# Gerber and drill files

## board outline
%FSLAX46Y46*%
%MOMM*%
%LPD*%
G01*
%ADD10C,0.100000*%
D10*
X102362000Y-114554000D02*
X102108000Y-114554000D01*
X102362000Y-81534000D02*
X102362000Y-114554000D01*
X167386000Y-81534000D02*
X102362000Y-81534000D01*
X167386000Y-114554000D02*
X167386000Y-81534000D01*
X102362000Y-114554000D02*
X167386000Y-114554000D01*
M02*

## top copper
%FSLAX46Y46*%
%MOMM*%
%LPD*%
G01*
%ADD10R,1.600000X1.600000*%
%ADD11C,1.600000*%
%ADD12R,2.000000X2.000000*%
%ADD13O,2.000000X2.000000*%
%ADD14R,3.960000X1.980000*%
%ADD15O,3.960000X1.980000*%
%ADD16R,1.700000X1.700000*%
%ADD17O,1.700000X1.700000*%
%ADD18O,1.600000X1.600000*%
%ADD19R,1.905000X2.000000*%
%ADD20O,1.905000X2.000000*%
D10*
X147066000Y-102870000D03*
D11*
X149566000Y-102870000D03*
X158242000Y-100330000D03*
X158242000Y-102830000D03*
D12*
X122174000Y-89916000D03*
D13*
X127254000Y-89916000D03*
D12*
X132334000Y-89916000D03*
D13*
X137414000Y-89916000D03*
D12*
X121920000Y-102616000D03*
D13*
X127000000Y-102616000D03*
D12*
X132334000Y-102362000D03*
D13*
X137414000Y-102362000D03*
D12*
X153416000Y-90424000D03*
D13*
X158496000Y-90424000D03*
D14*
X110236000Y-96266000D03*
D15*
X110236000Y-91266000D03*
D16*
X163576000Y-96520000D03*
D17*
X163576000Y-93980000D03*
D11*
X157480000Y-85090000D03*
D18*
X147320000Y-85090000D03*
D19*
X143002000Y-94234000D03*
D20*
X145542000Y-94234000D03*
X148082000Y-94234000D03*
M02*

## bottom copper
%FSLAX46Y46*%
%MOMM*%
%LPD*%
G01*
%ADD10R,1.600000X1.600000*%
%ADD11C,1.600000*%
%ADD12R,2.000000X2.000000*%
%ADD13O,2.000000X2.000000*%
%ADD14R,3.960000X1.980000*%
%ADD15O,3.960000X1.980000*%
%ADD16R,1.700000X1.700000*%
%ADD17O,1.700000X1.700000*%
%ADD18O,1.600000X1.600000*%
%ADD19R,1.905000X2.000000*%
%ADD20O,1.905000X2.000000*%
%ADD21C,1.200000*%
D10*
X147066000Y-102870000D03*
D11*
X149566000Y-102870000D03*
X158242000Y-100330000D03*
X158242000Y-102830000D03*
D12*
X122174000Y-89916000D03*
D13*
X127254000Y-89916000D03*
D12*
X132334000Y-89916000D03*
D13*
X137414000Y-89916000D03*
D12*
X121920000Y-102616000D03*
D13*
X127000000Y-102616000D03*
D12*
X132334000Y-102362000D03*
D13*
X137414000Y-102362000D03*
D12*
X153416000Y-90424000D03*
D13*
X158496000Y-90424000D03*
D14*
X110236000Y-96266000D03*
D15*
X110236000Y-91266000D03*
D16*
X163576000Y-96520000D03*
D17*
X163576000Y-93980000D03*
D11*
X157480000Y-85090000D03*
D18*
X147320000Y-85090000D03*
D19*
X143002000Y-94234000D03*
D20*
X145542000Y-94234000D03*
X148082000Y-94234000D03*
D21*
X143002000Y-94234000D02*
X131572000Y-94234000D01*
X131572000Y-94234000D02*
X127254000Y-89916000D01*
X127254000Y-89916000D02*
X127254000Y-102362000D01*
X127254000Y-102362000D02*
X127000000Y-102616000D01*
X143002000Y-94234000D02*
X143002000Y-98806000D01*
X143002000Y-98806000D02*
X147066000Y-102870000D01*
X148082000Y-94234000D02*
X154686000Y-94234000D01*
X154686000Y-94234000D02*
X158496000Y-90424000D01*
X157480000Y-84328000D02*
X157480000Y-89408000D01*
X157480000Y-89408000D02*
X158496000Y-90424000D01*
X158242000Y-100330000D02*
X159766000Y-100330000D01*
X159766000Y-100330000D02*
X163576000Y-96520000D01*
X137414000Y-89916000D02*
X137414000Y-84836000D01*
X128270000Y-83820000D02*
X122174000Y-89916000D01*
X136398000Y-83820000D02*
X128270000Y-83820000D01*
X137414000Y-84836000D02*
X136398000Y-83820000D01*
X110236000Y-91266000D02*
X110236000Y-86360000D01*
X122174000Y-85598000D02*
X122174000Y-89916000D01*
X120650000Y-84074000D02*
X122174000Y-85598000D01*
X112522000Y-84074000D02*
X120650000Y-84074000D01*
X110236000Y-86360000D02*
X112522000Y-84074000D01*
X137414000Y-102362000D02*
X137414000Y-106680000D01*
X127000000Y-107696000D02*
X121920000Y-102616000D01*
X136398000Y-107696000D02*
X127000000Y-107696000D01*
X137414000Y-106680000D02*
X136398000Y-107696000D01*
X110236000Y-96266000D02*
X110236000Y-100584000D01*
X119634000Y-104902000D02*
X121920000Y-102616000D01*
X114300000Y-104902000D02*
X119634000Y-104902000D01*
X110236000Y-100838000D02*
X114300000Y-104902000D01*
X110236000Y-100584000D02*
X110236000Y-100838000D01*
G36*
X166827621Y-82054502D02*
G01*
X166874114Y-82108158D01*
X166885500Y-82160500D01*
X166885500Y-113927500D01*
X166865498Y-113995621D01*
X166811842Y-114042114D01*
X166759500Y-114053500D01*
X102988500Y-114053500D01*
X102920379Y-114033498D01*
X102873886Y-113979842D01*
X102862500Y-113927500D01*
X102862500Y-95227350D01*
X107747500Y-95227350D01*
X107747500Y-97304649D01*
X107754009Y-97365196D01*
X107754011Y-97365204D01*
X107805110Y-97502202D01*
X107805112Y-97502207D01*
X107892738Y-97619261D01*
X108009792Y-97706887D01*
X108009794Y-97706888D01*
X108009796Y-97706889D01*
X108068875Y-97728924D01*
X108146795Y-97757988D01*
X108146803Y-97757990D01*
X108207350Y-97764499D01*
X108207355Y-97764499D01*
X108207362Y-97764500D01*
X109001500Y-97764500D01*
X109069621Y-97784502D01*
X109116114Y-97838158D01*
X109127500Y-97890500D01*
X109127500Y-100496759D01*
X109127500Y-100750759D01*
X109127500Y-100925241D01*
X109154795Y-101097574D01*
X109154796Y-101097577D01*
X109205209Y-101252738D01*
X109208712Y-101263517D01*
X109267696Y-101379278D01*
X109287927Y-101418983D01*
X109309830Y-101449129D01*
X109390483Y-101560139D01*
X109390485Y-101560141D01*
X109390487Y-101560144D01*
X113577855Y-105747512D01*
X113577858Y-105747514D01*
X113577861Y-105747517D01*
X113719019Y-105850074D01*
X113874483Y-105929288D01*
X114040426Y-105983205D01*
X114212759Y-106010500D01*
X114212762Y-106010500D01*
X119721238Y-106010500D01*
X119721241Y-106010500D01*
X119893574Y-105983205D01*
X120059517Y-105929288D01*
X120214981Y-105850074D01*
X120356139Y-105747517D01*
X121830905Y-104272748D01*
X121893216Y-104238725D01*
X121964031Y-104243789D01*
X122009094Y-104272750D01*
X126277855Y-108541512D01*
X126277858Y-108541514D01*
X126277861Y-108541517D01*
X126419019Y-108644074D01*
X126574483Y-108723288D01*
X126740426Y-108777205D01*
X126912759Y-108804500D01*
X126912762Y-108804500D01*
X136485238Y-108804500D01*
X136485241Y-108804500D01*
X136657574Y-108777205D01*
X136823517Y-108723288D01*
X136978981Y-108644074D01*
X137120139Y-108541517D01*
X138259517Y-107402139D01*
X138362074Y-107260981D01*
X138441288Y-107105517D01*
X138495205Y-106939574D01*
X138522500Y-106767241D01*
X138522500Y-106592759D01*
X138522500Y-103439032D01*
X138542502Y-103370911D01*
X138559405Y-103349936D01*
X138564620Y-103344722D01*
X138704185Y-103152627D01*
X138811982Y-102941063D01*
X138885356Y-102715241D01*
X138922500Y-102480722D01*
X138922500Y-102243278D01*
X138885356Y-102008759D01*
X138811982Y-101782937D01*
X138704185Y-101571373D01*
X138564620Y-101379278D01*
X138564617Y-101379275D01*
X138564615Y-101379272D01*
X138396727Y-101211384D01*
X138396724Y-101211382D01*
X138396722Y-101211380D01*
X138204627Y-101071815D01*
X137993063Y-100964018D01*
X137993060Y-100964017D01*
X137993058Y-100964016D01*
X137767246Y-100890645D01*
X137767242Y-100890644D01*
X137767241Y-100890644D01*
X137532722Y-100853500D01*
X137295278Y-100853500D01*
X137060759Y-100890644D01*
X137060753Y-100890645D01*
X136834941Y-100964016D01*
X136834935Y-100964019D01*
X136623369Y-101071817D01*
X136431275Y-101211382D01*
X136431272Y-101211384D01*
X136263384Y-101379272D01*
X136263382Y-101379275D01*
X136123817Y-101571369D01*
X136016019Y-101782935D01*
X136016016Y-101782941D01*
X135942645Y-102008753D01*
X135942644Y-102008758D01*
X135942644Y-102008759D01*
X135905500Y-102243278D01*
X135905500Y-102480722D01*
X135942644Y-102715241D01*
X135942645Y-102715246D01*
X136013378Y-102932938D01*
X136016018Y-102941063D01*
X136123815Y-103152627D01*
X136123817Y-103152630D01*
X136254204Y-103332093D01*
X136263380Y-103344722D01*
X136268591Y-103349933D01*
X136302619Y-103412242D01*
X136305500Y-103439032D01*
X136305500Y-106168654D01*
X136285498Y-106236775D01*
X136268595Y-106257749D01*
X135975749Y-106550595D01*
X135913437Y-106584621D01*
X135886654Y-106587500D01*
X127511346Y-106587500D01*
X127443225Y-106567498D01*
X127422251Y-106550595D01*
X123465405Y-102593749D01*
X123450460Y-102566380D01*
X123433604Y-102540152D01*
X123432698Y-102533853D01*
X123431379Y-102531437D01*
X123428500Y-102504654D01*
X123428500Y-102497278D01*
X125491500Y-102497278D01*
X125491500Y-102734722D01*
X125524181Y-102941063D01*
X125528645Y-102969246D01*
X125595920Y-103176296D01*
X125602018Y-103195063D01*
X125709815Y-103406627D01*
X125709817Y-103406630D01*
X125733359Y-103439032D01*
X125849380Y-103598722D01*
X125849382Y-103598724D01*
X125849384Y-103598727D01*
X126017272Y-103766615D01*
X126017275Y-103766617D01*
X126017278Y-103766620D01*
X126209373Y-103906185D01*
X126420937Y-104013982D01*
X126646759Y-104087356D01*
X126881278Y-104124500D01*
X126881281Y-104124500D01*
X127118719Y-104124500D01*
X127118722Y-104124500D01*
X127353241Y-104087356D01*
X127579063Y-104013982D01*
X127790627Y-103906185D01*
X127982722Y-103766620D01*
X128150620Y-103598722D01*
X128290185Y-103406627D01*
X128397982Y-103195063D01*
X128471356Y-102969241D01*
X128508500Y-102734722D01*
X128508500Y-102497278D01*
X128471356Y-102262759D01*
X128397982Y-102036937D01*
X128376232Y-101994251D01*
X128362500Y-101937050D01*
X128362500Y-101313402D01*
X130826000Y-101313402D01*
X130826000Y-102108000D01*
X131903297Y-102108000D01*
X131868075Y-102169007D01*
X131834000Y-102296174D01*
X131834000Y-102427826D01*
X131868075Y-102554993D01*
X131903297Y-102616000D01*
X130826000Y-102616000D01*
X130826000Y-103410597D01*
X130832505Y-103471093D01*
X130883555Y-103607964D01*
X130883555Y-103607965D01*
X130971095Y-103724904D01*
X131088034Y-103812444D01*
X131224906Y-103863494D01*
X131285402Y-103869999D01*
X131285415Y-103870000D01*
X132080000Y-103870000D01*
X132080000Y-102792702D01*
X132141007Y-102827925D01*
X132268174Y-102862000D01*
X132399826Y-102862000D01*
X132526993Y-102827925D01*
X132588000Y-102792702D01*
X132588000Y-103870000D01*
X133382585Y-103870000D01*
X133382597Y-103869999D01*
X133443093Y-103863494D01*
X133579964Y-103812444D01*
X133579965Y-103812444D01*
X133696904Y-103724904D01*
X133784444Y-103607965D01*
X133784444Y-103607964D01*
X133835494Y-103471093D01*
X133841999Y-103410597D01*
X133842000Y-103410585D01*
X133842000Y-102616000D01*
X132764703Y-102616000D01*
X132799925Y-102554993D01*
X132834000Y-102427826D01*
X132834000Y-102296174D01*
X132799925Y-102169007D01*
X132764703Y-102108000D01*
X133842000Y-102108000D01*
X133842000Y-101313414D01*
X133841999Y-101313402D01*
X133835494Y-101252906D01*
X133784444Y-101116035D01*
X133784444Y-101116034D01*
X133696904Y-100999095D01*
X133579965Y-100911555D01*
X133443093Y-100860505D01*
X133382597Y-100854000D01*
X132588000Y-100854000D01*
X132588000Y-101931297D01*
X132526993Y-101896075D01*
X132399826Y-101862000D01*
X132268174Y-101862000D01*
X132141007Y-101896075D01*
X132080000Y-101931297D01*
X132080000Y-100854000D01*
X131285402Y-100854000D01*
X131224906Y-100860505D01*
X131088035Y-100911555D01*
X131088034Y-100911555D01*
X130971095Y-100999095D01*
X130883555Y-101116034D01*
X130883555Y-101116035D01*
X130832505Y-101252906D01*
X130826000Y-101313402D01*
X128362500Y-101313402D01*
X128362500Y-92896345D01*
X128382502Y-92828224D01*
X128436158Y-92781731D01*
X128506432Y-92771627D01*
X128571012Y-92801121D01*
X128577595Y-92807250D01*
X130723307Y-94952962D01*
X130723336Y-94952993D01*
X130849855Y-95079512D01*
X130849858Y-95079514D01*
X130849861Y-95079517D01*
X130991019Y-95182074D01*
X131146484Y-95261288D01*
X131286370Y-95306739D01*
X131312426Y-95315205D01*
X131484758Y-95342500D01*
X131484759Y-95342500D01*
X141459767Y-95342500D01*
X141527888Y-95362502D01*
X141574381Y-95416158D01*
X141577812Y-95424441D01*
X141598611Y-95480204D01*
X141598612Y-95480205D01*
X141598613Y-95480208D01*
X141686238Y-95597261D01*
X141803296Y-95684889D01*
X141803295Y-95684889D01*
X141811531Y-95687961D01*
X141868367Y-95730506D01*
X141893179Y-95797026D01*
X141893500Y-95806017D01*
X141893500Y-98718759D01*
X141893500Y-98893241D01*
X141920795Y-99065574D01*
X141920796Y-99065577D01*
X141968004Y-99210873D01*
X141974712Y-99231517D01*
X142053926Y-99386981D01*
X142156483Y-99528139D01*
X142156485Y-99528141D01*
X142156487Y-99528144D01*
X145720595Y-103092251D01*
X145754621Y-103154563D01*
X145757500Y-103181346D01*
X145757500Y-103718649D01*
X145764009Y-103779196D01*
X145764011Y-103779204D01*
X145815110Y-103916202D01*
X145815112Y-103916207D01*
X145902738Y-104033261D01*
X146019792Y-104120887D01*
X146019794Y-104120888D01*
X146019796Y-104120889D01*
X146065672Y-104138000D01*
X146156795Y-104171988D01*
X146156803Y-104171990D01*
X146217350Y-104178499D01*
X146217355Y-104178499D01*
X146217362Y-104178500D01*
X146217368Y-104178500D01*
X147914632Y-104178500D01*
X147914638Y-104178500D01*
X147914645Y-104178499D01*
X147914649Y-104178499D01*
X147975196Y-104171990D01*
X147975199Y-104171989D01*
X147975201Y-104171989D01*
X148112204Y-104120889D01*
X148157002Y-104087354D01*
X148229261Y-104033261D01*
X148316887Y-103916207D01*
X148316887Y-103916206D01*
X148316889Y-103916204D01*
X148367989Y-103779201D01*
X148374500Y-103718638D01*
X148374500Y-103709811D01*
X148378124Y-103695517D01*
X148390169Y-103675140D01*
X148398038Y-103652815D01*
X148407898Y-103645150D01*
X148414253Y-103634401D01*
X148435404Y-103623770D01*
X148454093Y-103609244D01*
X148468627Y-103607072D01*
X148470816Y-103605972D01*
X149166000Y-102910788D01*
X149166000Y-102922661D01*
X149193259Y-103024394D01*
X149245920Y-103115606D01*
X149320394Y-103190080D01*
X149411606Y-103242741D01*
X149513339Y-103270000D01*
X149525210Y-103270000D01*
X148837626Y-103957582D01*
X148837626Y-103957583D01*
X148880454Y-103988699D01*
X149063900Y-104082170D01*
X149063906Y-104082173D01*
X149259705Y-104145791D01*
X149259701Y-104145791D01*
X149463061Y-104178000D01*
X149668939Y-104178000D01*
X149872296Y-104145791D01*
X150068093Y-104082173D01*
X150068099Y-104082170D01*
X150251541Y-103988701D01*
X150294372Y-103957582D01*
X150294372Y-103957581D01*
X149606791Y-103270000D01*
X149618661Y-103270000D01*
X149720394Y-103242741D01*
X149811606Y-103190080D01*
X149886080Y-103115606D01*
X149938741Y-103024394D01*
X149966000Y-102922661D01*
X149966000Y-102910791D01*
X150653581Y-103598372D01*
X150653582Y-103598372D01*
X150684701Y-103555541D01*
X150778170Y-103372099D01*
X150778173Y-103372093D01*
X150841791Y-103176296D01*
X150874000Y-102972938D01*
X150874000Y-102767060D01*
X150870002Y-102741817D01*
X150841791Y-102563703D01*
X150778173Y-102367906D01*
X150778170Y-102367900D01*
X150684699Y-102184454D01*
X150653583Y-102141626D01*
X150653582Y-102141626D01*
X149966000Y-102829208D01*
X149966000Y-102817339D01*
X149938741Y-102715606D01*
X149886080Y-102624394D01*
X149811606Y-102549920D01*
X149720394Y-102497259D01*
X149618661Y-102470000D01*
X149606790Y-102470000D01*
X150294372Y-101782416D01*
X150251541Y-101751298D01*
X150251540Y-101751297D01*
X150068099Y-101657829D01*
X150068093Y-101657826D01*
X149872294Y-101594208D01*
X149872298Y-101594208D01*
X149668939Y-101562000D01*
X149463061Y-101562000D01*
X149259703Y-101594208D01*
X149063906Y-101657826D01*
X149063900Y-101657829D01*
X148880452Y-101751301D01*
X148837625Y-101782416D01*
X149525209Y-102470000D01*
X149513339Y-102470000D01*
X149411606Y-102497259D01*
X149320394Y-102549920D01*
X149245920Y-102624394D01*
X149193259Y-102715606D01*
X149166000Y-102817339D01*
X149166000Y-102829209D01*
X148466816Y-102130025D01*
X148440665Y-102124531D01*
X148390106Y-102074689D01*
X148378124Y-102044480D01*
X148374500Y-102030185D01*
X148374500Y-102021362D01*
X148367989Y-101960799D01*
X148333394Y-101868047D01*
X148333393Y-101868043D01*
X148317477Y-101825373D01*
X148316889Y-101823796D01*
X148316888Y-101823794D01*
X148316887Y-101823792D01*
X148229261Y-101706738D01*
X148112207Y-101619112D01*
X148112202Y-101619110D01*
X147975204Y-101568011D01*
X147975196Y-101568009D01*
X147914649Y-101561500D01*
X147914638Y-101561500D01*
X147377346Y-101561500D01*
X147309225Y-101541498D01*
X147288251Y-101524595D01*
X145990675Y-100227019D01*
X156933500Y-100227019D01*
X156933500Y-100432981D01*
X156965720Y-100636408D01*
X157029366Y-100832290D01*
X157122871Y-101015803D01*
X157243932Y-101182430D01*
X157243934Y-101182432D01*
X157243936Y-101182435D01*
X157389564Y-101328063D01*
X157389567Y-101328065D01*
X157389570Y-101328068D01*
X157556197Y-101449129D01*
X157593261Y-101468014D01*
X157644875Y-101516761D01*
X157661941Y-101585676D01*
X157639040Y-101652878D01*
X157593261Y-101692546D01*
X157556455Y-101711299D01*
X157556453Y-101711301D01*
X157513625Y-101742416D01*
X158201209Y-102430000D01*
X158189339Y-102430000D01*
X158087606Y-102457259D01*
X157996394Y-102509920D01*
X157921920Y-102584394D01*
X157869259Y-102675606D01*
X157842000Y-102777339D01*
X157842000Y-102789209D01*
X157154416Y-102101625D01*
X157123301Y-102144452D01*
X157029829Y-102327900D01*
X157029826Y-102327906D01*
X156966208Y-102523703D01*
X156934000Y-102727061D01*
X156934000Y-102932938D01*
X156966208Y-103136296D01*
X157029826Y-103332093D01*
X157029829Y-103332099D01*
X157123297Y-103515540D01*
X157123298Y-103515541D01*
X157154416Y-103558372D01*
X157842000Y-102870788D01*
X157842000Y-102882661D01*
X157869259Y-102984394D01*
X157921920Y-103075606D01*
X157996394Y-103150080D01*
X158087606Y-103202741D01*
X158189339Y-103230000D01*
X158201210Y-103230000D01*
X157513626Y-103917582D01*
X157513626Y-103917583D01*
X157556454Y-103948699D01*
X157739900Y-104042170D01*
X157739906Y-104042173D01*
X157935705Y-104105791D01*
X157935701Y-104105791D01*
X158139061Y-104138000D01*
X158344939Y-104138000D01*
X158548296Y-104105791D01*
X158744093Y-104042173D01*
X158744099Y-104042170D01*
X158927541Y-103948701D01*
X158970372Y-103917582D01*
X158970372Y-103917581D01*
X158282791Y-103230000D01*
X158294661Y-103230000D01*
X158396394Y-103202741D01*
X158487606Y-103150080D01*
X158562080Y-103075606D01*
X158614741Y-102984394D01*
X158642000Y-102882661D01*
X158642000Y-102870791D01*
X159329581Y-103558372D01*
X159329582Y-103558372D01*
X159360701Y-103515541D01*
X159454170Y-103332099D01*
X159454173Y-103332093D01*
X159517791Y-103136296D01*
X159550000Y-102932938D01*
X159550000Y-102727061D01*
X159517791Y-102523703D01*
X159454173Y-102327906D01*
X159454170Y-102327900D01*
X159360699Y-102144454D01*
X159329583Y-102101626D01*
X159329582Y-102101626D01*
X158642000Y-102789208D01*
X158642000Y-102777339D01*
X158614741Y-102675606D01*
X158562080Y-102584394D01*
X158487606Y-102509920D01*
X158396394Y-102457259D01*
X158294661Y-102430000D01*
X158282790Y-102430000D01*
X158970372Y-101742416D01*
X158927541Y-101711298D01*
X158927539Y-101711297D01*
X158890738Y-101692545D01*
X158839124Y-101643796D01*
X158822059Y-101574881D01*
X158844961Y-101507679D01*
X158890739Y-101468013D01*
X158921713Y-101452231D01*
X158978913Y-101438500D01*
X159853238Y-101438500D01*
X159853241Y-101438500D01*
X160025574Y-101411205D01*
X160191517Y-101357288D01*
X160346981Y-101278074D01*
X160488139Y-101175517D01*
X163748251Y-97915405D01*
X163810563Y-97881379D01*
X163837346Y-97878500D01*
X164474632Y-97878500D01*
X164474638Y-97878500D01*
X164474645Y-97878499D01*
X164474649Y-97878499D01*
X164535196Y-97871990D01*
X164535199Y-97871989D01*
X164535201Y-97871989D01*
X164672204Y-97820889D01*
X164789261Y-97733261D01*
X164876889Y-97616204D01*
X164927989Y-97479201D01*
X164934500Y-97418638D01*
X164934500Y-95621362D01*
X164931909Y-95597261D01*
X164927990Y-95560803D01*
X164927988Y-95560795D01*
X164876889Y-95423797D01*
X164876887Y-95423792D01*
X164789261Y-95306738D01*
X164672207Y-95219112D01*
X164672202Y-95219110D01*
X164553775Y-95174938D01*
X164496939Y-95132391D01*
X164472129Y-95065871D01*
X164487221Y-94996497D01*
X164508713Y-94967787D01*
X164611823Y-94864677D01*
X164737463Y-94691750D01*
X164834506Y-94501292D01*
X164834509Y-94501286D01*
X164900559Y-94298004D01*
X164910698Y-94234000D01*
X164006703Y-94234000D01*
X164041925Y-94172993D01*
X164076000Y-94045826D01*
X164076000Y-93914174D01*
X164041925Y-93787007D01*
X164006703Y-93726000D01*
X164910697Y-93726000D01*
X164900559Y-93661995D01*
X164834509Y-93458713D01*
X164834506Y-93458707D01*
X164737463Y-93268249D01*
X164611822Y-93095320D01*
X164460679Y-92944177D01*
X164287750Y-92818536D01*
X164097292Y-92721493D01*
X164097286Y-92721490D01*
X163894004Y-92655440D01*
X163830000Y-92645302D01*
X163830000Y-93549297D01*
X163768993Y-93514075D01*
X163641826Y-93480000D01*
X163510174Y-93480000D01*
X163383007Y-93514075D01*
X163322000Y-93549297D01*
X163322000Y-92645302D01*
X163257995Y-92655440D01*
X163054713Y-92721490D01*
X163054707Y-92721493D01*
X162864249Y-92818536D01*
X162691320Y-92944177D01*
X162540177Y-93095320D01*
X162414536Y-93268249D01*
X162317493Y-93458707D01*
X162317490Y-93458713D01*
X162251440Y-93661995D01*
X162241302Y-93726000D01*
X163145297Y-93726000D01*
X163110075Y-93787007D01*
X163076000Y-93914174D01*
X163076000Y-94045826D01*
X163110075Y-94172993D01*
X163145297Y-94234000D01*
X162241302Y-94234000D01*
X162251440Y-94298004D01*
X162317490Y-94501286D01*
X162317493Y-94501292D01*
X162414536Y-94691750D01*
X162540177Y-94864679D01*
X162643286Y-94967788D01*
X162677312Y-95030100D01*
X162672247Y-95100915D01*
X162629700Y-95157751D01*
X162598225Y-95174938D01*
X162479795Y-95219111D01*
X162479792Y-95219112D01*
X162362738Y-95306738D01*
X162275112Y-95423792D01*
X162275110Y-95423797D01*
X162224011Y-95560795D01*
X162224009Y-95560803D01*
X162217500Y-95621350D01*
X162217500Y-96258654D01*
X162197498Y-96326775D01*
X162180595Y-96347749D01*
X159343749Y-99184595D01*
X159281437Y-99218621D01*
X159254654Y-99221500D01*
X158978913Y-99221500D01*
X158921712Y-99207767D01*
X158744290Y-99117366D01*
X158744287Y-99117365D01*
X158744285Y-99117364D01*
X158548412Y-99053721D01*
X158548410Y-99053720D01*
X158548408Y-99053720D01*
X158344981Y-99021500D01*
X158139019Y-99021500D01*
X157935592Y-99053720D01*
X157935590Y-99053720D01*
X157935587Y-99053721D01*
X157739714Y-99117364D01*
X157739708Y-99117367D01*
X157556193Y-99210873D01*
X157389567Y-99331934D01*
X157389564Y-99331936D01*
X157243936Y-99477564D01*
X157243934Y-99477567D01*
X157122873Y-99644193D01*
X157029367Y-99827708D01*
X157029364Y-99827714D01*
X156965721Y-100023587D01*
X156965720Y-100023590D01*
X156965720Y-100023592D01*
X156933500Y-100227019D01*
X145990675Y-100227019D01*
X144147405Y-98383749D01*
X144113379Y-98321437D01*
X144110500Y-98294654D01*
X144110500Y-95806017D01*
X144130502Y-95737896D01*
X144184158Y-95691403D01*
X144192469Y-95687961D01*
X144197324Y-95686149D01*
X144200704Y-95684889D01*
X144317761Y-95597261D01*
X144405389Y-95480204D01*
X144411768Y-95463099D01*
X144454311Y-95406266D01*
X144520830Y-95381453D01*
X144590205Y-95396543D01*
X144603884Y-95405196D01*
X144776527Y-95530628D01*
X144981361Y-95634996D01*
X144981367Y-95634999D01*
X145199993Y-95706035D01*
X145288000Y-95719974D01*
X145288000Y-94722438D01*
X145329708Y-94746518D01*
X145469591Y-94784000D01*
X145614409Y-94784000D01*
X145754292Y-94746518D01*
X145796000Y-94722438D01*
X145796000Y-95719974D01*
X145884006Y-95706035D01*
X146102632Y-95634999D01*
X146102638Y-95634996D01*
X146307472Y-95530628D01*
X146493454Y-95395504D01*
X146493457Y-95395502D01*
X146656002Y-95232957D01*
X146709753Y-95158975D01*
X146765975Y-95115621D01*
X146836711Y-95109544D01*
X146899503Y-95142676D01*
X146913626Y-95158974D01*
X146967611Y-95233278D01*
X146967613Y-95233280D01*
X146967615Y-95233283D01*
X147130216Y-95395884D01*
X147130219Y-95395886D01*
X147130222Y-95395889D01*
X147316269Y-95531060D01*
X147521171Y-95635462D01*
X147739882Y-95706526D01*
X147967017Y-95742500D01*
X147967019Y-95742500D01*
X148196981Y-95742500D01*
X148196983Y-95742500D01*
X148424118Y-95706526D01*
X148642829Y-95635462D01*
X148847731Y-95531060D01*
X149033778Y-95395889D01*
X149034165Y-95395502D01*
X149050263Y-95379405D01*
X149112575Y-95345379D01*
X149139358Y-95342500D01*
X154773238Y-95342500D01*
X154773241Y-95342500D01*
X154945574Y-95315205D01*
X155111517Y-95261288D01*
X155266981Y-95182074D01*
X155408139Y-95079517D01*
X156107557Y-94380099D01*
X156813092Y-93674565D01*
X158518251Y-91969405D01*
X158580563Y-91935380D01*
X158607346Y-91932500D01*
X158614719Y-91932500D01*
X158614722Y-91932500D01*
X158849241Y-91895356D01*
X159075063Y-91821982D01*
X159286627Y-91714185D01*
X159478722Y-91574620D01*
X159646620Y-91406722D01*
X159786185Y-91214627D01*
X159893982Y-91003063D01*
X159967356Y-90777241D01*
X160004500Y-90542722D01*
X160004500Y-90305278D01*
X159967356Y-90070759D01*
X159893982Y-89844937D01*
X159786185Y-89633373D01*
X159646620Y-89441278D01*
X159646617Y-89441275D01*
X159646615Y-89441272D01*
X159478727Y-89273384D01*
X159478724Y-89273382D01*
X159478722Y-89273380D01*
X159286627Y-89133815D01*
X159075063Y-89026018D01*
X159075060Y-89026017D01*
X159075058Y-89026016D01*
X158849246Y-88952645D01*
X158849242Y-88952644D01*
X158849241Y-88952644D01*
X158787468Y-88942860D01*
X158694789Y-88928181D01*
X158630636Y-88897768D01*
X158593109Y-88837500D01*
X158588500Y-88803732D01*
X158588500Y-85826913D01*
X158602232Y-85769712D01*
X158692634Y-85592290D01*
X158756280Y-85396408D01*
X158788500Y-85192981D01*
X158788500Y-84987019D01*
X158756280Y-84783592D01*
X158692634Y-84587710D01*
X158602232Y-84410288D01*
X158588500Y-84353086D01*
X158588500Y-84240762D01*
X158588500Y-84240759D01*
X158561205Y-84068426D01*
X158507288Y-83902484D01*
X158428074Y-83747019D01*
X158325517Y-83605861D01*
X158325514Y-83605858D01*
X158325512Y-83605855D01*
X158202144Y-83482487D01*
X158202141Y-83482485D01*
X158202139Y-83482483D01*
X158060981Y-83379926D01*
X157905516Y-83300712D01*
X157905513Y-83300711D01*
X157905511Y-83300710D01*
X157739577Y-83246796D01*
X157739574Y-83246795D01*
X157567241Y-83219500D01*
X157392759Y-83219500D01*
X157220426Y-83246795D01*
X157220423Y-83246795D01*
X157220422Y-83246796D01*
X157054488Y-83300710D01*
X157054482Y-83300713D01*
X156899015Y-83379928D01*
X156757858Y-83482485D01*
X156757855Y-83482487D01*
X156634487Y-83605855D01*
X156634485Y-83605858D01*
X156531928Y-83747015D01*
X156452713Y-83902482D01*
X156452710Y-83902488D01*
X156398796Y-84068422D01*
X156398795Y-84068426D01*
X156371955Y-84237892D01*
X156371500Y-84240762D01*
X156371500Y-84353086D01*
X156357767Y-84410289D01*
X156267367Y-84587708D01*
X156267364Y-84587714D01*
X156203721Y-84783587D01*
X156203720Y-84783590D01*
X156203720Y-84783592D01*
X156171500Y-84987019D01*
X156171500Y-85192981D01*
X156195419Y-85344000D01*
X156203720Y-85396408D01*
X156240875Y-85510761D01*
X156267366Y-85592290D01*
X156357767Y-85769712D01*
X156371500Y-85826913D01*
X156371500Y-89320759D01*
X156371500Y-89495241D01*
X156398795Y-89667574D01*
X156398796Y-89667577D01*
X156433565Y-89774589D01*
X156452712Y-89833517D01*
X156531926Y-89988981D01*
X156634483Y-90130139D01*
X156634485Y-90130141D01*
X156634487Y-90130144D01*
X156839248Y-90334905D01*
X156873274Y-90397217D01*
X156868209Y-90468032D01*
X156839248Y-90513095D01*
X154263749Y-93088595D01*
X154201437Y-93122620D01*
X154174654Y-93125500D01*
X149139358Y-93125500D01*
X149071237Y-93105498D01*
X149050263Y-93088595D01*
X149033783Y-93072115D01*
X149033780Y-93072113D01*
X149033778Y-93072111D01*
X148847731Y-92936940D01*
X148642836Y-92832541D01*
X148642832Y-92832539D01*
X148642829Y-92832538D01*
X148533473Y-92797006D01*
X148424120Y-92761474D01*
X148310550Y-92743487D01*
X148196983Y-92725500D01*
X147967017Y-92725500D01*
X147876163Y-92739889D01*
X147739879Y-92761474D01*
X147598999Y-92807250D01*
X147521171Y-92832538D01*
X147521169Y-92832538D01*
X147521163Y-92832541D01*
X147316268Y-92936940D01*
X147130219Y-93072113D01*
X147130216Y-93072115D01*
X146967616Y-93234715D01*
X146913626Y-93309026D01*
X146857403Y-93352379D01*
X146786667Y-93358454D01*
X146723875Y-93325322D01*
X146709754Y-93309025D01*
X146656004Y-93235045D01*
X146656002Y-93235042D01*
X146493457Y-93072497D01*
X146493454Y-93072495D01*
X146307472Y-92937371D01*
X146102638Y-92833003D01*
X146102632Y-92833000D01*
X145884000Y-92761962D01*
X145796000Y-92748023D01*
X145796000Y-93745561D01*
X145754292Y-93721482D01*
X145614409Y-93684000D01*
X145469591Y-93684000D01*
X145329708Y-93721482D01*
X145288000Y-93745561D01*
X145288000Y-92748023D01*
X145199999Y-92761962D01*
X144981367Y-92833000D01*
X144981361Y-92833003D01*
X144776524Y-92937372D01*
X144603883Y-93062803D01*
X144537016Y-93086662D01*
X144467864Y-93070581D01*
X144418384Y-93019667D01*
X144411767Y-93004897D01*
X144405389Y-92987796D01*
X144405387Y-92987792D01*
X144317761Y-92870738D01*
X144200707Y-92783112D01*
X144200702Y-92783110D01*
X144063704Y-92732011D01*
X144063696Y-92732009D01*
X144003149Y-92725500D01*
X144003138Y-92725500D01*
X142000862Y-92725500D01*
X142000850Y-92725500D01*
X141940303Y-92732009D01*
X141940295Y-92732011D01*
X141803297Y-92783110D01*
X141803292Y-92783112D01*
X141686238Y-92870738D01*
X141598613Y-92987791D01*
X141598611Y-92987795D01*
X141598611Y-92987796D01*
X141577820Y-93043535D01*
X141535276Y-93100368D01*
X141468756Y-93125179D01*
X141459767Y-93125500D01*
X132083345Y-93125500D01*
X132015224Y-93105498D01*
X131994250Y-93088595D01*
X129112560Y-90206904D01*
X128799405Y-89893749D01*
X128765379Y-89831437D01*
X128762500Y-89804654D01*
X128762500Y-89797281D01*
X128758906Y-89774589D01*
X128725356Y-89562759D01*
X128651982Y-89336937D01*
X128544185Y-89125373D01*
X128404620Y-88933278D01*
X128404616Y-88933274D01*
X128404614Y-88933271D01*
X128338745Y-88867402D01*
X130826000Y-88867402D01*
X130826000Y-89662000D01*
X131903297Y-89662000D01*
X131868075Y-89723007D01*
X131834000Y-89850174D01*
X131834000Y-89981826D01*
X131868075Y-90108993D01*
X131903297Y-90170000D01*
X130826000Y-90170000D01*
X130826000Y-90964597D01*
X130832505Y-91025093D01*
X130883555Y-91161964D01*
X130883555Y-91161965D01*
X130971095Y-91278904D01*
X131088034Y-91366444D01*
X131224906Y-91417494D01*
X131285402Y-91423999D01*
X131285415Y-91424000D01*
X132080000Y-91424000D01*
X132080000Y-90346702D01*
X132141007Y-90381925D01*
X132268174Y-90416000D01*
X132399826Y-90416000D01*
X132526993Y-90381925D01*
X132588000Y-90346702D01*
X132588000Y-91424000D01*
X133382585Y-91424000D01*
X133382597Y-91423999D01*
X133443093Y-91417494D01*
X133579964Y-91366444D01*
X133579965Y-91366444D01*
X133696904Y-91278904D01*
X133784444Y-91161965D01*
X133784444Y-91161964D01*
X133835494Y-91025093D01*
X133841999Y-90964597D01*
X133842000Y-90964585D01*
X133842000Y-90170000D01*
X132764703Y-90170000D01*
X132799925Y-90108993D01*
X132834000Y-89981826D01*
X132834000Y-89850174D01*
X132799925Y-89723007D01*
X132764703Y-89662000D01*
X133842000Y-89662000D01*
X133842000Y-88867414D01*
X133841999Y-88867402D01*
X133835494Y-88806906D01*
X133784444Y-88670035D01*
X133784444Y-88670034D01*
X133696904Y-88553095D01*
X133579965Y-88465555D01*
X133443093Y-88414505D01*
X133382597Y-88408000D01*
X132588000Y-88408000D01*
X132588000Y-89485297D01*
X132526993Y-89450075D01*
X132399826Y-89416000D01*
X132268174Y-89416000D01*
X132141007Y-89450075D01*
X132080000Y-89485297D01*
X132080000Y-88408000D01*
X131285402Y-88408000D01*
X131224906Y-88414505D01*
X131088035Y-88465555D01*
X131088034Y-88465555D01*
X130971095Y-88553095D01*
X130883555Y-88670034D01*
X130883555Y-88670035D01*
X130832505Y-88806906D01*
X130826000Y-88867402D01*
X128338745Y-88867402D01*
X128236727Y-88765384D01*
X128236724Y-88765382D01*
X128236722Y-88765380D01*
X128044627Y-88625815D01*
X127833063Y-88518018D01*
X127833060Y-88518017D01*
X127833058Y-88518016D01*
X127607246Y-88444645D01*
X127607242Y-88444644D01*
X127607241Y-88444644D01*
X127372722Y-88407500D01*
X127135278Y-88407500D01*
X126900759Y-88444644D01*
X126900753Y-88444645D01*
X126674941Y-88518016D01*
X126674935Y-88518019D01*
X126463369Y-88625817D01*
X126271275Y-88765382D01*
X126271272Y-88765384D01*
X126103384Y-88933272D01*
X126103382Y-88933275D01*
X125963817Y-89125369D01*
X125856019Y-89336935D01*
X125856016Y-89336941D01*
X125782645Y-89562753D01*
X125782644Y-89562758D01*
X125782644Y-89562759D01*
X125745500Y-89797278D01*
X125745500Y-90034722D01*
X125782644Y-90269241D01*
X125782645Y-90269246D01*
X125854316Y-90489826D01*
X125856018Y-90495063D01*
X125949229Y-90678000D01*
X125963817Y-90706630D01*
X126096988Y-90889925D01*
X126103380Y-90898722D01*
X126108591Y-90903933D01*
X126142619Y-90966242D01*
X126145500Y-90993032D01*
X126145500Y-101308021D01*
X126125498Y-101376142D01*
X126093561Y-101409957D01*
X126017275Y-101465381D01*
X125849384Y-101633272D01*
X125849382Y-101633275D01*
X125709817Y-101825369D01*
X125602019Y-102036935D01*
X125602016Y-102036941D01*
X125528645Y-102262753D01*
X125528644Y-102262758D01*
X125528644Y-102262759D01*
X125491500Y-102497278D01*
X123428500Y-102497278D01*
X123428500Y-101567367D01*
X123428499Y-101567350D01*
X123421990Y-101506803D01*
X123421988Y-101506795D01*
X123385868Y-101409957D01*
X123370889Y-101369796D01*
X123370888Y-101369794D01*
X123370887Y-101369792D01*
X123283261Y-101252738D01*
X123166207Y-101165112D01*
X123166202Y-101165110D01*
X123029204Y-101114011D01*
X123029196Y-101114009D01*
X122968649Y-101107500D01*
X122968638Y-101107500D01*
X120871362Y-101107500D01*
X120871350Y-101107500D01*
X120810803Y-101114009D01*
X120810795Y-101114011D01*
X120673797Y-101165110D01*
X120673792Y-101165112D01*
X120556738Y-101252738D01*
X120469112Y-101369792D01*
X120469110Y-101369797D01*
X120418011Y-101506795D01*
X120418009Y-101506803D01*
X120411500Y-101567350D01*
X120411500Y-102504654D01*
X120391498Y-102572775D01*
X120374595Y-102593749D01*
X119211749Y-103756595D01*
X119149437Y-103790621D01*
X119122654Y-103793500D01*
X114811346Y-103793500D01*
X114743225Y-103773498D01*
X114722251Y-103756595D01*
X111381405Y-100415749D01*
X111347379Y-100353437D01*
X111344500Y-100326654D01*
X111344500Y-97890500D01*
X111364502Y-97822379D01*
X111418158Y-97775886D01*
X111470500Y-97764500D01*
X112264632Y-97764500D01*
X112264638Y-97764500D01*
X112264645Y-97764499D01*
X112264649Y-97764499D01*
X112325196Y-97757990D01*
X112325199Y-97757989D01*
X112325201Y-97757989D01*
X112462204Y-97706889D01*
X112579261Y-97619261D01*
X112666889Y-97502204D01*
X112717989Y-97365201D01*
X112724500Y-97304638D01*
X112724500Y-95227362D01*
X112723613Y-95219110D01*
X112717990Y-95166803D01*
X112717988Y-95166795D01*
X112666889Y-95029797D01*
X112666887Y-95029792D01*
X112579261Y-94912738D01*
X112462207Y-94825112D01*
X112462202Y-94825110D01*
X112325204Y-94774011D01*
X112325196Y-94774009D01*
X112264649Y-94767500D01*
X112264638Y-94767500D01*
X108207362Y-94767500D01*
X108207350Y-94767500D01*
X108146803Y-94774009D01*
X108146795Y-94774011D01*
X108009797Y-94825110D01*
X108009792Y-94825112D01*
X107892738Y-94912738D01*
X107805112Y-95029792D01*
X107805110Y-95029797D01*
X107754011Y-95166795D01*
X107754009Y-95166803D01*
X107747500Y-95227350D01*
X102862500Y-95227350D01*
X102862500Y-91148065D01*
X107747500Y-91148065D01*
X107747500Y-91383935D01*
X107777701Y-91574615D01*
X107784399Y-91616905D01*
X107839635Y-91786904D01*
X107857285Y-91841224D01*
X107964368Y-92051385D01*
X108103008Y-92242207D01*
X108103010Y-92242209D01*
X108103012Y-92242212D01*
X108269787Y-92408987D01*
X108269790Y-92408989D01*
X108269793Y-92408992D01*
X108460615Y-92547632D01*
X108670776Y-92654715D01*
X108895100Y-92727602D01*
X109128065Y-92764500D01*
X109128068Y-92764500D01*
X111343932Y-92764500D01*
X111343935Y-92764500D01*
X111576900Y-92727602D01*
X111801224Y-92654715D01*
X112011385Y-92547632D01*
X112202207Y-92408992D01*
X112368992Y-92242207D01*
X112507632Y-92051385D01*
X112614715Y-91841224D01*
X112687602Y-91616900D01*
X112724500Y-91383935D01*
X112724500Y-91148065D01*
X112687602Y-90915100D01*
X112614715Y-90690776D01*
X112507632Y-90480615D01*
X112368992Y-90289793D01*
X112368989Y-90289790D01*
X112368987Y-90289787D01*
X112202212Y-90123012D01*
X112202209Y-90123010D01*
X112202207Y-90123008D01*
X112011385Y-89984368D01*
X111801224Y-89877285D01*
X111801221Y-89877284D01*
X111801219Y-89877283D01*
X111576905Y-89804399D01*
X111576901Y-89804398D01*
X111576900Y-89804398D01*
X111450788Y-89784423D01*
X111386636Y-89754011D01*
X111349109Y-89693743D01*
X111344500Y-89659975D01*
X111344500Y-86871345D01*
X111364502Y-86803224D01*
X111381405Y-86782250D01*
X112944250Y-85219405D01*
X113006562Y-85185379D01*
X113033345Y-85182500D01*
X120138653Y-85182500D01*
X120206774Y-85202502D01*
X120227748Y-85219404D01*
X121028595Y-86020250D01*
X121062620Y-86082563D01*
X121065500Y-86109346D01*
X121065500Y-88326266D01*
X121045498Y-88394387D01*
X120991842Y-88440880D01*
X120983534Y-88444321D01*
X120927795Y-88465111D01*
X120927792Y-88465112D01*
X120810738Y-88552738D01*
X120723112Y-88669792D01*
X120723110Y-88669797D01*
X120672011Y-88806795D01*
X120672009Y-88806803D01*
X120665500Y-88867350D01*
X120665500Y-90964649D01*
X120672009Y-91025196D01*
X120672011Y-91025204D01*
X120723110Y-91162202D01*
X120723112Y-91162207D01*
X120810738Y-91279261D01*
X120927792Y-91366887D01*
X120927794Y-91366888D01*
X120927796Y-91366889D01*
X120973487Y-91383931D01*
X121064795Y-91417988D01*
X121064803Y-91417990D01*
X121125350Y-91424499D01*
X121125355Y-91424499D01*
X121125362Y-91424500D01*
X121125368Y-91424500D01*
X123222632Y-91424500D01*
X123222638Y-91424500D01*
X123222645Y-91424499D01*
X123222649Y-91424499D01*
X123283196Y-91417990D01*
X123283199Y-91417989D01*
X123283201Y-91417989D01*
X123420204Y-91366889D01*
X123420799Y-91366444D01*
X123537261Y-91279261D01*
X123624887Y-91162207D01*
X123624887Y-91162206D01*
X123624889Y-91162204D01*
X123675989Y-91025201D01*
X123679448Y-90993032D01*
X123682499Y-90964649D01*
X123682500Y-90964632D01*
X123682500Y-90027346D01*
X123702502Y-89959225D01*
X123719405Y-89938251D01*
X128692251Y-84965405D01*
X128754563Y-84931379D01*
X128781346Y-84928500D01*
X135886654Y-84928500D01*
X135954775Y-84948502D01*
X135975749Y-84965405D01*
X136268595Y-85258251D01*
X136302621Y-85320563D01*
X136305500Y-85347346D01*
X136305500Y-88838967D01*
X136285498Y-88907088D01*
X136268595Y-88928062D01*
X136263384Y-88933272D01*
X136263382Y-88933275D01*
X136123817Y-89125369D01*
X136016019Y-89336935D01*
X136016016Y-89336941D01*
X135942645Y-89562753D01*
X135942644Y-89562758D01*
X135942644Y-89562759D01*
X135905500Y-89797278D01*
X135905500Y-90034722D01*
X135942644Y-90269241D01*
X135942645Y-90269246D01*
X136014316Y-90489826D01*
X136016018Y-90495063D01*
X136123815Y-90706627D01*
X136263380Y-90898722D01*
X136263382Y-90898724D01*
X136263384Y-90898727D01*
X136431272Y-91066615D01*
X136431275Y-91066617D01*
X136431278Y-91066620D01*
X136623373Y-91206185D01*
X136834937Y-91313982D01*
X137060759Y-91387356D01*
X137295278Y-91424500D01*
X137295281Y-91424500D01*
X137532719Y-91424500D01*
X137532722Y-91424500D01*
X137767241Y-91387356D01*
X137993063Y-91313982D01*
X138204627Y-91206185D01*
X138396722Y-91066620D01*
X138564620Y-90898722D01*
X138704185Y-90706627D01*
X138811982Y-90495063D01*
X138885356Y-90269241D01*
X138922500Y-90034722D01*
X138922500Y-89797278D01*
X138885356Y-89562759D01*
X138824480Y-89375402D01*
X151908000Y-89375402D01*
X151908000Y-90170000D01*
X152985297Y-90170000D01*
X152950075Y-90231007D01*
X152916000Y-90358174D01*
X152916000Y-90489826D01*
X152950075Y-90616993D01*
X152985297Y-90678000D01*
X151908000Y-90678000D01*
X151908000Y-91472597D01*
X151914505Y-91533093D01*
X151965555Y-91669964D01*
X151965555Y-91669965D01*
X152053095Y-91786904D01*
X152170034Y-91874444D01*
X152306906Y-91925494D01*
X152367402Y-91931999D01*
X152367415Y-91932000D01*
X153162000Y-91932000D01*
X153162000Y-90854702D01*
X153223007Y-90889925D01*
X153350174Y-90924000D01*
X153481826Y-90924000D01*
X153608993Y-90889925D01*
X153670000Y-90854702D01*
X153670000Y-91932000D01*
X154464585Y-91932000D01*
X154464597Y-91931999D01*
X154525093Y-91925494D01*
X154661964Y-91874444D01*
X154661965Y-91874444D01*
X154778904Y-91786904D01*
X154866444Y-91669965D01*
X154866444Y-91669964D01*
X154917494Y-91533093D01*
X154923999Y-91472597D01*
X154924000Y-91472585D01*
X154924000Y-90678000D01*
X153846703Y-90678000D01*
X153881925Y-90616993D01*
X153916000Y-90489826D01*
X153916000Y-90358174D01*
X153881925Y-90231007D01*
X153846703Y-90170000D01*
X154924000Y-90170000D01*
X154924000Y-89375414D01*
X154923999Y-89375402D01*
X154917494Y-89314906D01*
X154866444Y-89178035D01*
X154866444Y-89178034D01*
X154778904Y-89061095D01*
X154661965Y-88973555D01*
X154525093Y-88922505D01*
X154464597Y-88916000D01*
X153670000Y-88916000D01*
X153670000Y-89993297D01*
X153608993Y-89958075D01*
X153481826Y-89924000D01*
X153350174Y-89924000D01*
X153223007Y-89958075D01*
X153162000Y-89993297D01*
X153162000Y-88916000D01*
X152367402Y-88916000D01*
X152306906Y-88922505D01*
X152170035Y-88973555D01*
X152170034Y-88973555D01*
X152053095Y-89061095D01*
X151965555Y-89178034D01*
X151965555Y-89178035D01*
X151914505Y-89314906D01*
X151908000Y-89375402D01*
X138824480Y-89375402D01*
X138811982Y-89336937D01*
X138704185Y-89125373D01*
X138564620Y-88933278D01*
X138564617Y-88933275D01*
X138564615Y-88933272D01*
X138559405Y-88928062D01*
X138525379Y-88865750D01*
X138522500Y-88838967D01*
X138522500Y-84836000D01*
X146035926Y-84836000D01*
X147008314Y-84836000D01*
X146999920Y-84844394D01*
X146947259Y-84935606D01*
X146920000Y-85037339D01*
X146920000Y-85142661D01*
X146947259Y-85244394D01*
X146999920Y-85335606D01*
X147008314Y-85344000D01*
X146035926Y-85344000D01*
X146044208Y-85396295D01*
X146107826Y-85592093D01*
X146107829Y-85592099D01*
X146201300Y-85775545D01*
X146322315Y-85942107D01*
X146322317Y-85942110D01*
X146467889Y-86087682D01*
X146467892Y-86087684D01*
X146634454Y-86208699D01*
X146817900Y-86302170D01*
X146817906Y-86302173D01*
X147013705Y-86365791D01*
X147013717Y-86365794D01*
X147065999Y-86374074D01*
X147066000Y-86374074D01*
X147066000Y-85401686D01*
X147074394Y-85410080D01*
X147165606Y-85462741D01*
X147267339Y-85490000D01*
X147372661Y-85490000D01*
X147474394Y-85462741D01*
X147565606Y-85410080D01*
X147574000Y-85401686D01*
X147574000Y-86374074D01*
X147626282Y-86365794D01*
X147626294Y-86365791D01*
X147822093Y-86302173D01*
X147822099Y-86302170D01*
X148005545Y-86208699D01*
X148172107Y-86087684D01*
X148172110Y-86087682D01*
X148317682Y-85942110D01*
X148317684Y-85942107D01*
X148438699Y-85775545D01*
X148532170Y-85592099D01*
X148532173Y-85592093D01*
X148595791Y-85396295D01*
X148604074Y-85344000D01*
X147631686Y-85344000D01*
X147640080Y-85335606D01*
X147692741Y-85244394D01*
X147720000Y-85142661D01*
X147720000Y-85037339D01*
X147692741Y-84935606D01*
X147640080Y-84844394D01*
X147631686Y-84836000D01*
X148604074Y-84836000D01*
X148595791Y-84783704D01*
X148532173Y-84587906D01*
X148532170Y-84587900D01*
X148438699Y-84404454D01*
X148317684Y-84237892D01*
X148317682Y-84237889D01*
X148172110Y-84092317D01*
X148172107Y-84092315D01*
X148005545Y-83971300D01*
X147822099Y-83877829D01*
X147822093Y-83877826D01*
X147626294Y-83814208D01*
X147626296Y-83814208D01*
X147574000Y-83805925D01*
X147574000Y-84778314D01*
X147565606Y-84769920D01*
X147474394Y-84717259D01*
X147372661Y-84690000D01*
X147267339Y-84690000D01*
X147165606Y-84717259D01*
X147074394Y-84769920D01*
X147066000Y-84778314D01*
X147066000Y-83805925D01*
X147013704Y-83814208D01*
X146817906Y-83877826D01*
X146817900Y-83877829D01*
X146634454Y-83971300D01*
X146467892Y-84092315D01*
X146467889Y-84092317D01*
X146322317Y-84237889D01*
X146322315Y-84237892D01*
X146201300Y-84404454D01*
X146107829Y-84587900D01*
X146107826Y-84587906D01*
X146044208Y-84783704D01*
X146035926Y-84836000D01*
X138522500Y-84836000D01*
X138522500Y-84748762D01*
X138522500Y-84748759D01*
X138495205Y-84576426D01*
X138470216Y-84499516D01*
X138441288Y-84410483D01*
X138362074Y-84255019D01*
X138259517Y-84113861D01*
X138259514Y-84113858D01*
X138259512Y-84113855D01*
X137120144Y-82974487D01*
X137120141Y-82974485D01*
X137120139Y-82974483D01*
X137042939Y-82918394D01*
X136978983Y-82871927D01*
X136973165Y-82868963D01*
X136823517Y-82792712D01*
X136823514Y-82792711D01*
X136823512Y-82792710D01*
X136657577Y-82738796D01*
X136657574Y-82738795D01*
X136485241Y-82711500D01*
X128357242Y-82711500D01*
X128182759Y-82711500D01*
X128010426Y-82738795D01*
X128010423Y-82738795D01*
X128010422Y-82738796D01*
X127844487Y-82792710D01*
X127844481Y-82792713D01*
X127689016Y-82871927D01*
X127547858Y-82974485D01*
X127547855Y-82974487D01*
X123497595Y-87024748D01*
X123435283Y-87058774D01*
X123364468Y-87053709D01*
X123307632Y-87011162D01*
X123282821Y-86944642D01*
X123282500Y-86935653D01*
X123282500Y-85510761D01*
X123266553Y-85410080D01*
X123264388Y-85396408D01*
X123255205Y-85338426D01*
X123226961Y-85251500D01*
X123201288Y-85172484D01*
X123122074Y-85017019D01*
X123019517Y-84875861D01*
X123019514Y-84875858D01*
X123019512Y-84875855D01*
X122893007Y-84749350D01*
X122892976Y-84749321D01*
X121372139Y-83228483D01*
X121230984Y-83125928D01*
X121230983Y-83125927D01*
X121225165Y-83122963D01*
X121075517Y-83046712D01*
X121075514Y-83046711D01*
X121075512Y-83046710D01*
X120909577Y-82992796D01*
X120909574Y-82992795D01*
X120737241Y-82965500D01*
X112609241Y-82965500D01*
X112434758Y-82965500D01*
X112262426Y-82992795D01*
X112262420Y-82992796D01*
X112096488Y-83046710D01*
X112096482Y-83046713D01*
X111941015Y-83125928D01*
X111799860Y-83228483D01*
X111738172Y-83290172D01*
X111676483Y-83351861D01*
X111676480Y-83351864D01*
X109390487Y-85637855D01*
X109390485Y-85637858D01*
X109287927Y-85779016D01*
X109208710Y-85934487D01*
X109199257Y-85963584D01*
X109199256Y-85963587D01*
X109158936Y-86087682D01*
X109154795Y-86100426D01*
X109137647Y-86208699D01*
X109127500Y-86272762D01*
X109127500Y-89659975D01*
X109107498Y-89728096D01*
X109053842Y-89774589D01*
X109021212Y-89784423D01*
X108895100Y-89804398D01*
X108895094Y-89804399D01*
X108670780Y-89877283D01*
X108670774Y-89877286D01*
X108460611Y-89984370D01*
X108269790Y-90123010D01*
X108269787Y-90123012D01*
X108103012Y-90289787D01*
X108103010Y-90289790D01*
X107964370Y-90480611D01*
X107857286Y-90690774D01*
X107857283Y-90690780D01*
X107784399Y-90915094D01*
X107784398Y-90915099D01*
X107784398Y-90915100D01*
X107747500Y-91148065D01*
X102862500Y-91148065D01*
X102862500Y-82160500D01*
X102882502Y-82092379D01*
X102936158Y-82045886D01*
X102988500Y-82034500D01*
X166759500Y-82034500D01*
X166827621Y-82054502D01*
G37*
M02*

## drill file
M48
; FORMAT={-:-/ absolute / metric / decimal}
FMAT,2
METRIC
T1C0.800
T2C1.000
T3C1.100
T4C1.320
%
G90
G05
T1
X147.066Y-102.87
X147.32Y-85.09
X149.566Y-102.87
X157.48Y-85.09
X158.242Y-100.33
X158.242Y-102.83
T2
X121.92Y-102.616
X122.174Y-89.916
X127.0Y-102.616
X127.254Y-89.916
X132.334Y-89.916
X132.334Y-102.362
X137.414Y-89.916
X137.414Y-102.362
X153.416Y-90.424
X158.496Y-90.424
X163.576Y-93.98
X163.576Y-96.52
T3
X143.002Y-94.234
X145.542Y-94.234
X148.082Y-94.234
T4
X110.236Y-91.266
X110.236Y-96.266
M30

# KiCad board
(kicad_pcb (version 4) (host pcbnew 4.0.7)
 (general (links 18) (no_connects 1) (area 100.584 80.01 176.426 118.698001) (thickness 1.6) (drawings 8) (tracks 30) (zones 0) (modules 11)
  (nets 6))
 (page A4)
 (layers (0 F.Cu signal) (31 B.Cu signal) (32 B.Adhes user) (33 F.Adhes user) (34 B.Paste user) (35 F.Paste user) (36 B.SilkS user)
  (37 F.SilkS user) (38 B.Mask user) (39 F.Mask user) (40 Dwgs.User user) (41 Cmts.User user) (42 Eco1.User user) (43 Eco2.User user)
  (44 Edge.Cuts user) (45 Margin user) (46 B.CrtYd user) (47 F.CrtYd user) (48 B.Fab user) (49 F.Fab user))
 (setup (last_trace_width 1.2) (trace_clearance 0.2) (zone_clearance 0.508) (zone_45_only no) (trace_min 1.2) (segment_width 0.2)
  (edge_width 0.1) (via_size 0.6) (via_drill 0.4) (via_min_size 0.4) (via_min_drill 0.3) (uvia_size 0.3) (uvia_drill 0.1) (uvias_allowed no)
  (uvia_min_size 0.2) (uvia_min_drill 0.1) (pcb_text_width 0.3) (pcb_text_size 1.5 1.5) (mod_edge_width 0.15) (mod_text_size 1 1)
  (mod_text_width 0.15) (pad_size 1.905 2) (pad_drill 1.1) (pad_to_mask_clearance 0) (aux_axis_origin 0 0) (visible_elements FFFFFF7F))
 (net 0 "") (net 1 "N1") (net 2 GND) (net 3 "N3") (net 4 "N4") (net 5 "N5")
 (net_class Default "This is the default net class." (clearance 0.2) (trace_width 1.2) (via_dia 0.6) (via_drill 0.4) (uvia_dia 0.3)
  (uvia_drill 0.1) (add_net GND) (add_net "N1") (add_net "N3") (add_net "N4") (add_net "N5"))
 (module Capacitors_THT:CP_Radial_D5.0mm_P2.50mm (layer F.Cu) (at 147.066 102.87)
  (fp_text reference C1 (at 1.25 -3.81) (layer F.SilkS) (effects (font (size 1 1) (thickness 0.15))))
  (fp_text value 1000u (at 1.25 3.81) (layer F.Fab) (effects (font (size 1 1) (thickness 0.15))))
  (pad 1 thru_hole rect (at 0 0) (size 1.6 1.6) (drill 0.8) (layers *.Cu *.Mask) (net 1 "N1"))
  (pad 2 thru_hole circle (at 2.5 0) (size 1.6 1.6) (drill 0.8) (layers *.Cu *.Mask) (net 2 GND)))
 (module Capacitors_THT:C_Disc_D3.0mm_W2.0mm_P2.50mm (layer F.Cu) (at 158.242 100.33 270)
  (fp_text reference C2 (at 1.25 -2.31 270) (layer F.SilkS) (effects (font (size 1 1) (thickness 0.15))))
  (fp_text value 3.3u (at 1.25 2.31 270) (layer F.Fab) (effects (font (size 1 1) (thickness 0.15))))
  (pad 1 thru_hole circle (at 0 0 270) (size 1.6 1.6) (drill 0.8) (layers *.Cu *.Mask) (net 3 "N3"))
  (pad 2 thru_hole circle (at 2.5 0 270) (size 1.6 1.6) (drill 0.8) (layers *.Cu *.Mask) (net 2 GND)))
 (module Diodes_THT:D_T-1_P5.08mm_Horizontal (layer F.Cu) (at 122.174 89.916)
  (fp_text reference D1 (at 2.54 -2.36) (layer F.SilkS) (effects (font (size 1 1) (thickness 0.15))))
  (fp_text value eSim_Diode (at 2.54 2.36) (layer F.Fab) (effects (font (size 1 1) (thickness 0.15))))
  (pad 1 thru_hole rect (at 0 0) (size 2 2) (drill 1) (layers *.Cu *.Mask) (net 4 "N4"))
  (pad 2 thru_hole oval (at 5.08 0) (size 2 2) (drill 1) (layers *.Cu *.Mask) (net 1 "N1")))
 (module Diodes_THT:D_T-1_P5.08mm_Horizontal (layer F.Cu) (at 132.334 89.916)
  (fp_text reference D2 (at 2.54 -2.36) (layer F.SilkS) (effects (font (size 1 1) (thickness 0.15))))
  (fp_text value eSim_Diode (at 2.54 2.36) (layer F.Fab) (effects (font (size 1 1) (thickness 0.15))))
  (pad 1 thru_hole rect (at 0 0) (size 2 2) (drill 1) (layers *.Cu *.Mask) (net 2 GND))
  (pad 2 thru_hole oval (at 5.08 0) (size 2 2) (drill 1) (layers *.Cu *.Mask) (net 4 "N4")))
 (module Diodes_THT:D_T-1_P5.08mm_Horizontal (layer F.Cu) (at 121.92 102.616)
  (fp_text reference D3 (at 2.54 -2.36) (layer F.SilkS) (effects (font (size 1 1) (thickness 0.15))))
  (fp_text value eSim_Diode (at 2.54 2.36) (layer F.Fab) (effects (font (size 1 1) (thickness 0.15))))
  (pad 1 thru_hole rect (at 0 0) (size 2 2) (drill 1) (layers *.Cu *.Mask) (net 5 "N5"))
  (pad 2 thru_hole oval (at 5.08 0) (size 2 2) (drill 1) (layers *.Cu *.Mask) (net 1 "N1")))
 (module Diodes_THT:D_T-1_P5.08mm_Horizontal (layer F.Cu) (at 132.334 102.362)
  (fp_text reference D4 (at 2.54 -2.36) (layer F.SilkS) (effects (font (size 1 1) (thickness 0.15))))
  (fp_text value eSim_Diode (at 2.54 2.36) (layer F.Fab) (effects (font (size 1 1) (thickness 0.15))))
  (pad 1 thru_hole rect (at 0 0) (size 2 2) (drill 1) (layers *.Cu *.Mask) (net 2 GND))
  (pad 2 thru_hole oval (at 5.08 0) (size 2 2) (drill 1) (layers *.Cu *.Mask) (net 5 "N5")))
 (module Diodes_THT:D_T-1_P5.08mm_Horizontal (layer F.Cu) (at 153.416 90.424)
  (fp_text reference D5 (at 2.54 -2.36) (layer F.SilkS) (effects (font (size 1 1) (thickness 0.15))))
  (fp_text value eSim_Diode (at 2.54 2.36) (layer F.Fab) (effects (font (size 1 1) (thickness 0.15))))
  (pad 1 thru_hole rect (at 0 0) (size 2 2) (drill 1) (layers *.Cu *.Mask) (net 2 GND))
  (pad 2 thru_hole oval (at 5.08 0) (size 2 2) (drill 1) (layers *.Cu *.Mask) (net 3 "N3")))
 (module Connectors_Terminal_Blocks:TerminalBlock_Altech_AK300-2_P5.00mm (layer F.Cu) (at 110.236 96.266 90)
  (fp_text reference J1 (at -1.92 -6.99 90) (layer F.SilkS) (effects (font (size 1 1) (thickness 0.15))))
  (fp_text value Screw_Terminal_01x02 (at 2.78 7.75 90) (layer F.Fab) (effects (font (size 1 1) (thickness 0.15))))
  (pad 1 thru_hole rect (at 0 0 90) (size 1.98 3.96) (drill 1.32) (layers *.Cu *.Mask) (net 5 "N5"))
  (pad 2 thru_hole oval (at 5 0 90) (size 1.98 3.96) (drill 1.32) (layers *.Cu *.Mask) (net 4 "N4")))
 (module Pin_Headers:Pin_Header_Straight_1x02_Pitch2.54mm (layer F.Cu) (at 163.576 96.52 180)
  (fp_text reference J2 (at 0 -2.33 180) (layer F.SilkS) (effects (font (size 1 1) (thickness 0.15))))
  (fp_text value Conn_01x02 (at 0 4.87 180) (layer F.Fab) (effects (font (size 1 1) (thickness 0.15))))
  (pad 1 thru_hole rect (at 0 0 180) (size 1.7 1.7) (drill 1) (layers *.Cu *.Mask) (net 3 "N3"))
  (pad 2 thru_hole oval (at 0 2.54 180) (size 1.7 1.7) (drill 1) (layers *.Cu *.Mask) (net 2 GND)))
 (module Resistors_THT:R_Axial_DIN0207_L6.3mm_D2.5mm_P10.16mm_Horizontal (layer F.Cu) (at 157.48 85.09 180)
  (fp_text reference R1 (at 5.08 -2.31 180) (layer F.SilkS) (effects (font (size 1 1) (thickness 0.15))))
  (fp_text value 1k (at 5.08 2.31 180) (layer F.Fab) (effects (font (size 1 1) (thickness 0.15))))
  (pad 1 thru_hole circle (at 0 0 180) (size 1.6 1.6) (drill 0.8) (layers *.Cu *.Mask) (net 3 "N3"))
  (pad 2 thru_hole oval (at 10.16 0 180) (size 1.6 1.6) (drill 0.8) (layers *.Cu *.Mask) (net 2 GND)))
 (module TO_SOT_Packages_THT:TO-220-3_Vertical (layer F.Cu) (at 143.002 94.234)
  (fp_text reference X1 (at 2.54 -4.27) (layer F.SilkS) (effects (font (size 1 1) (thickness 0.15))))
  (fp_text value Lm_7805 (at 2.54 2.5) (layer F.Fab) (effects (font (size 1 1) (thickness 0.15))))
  (pad 1 thru_hole rect (at 0 0) (size 1.905 2) (drill 1.1) (layers *.Cu *.Mask) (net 1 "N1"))
  (pad 2 thru_hole oval (at 2.54 0) (size 1.905 2) (drill 1.1) (layers *.Cu *.Mask) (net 2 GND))
  (pad 3 thru_hole oval (at 5.08 0) (size 1.905 2) (drill 1.1) (layers *.Cu *.Mask) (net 3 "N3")))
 (gr_line (start 102.362 114.554) (end 102.108 114.554) (angle 90) (layer Edge.Cuts) (width 0.1))
 (gr_line (start 102.362 81.534) (end 102.362 114.554) (angle 90) (layer Edge.Cuts) (width 0.1))
 (gr_line (start 167.386 81.534) (end 102.362 81.534) (angle 90) (layer Edge.Cuts) (width 0.1))
 (gr_line (start 167.386 114.554) (end 167.386 81.534) (angle 90) (layer Edge.Cuts) (width 0.1))
 (gr_line (start 102.362 114.554) (end 167.386 114.554) (angle 90) (layer Edge.Cuts) (width 0.1))
 (segment (start 143.002 94.234) (end 131.572 94.234) (width 1.2) (layer B.Cu) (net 1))
 (segment (start 131.572 94.234) (end 127.254 89.916) (width 1.2) (layer B.Cu) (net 1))
 (segment (start 127.254 89.916) (end 127.254 102.362) (width 1.2) (layer B.Cu) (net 1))
 (segment (start 127.254 102.362) (end 127 102.616) (width 1.2) (layer B.Cu) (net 1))
 (segment (start 143.002 94.234) (end 143.002 98.806) (width 1.2) (layer B.Cu) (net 1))
 (segment (start 143.002 98.806) (end 147.066 102.87) (width 1.2) (layer B.Cu) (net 1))
 (segment (start 148.082 94.234) (end 154.686 94.234) (width 1.2) (layer B.Cu) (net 3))
 (segment (start 154.686 94.234) (end 158.496 90.424) (width 1.2) (layer B.Cu) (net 3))
 (segment (start 157.48 84.328) (end 157.48 89.408) (width 1.2) (layer B.Cu) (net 3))
 (segment (start 157.48 89.408) (end 158.496 90.424) (width 1.2) (layer B.Cu) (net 3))
 (segment (start 158.242 100.33) (end 159.766 100.33) (width 1.2) (layer B.Cu) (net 3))
 (segment (start 159.766 100.33) (end 163.576 96.52) (width 1.2) (layer B.Cu) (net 3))
 (segment (start 137.414 89.916) (end 137.414 84.836) (width 1.2) (layer B.Cu) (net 4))
 (segment (start 128.27 83.82) (end 122.174 89.916) (width 1.2) (layer B.Cu) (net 4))
 (segment (start 136.398 83.82) (end 128.27 83.82) (width 1.2) (layer B.Cu) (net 4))
 (segment (start 137.414 84.836) (end 136.398 83.82) (width 1.2) (layer B.Cu) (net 4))
 (segment (start 110.236 91.266) (end 110.236 86.36) (width 1.2) (layer B.Cu) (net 4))
 (segment (start 122.174 85.598) (end 122.174 89.916) (width 1.2) (layer B.Cu) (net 4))
 (segment (start 120.65 84.074) (end 122.174 85.598) (width 1.2) (layer B.Cu) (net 4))
 (segment (start 112.522 84.074) (end 120.65 84.074) (width 1.2) (layer B.Cu) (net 4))
 (segment (start 110.236 86.36) (end 112.522 84.074) (width 1.2) (layer B.Cu) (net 4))
 (segment (start 137.414 102.362) (end 137.414 106.68) (width 1.2) (layer B.Cu) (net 5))
 (segment (start 127 107.696) (end 121.92 102.616) (width 1.2) (layer B.Cu) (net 5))
 (segment (start 136.398 107.696) (end 127 107.696) (width 1.2) (layer B.Cu) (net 5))
 (segment (start 137.414 106.68) (end 136.398 107.696) (width 1.2) (layer B.Cu) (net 5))
 (segment (start 110.236 96.266) (end 110.236 100.584) (width 1.2) (layer B.Cu) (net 5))
 (segment (start 119.634 104.902) (end 121.92 102.616) (width 1.2) (layer B.Cu) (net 5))
 (segment (start 114.3 104.902) (end 119.634 104.902) (width 1.2) (layer B.Cu) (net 5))
 (segment (start 110.236 100.838) (end 114.3 104.902) (width 1.2) (layer B.Cu) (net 5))
 (segment (start 110.236 100.584) (end 110.236 100.838) (width 1.2) (layer B.Cu) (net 5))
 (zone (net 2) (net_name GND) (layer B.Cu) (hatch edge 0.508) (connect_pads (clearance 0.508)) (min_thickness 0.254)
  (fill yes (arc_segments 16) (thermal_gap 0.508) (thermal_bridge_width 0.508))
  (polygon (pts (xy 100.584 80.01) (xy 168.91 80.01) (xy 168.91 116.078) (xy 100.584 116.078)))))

